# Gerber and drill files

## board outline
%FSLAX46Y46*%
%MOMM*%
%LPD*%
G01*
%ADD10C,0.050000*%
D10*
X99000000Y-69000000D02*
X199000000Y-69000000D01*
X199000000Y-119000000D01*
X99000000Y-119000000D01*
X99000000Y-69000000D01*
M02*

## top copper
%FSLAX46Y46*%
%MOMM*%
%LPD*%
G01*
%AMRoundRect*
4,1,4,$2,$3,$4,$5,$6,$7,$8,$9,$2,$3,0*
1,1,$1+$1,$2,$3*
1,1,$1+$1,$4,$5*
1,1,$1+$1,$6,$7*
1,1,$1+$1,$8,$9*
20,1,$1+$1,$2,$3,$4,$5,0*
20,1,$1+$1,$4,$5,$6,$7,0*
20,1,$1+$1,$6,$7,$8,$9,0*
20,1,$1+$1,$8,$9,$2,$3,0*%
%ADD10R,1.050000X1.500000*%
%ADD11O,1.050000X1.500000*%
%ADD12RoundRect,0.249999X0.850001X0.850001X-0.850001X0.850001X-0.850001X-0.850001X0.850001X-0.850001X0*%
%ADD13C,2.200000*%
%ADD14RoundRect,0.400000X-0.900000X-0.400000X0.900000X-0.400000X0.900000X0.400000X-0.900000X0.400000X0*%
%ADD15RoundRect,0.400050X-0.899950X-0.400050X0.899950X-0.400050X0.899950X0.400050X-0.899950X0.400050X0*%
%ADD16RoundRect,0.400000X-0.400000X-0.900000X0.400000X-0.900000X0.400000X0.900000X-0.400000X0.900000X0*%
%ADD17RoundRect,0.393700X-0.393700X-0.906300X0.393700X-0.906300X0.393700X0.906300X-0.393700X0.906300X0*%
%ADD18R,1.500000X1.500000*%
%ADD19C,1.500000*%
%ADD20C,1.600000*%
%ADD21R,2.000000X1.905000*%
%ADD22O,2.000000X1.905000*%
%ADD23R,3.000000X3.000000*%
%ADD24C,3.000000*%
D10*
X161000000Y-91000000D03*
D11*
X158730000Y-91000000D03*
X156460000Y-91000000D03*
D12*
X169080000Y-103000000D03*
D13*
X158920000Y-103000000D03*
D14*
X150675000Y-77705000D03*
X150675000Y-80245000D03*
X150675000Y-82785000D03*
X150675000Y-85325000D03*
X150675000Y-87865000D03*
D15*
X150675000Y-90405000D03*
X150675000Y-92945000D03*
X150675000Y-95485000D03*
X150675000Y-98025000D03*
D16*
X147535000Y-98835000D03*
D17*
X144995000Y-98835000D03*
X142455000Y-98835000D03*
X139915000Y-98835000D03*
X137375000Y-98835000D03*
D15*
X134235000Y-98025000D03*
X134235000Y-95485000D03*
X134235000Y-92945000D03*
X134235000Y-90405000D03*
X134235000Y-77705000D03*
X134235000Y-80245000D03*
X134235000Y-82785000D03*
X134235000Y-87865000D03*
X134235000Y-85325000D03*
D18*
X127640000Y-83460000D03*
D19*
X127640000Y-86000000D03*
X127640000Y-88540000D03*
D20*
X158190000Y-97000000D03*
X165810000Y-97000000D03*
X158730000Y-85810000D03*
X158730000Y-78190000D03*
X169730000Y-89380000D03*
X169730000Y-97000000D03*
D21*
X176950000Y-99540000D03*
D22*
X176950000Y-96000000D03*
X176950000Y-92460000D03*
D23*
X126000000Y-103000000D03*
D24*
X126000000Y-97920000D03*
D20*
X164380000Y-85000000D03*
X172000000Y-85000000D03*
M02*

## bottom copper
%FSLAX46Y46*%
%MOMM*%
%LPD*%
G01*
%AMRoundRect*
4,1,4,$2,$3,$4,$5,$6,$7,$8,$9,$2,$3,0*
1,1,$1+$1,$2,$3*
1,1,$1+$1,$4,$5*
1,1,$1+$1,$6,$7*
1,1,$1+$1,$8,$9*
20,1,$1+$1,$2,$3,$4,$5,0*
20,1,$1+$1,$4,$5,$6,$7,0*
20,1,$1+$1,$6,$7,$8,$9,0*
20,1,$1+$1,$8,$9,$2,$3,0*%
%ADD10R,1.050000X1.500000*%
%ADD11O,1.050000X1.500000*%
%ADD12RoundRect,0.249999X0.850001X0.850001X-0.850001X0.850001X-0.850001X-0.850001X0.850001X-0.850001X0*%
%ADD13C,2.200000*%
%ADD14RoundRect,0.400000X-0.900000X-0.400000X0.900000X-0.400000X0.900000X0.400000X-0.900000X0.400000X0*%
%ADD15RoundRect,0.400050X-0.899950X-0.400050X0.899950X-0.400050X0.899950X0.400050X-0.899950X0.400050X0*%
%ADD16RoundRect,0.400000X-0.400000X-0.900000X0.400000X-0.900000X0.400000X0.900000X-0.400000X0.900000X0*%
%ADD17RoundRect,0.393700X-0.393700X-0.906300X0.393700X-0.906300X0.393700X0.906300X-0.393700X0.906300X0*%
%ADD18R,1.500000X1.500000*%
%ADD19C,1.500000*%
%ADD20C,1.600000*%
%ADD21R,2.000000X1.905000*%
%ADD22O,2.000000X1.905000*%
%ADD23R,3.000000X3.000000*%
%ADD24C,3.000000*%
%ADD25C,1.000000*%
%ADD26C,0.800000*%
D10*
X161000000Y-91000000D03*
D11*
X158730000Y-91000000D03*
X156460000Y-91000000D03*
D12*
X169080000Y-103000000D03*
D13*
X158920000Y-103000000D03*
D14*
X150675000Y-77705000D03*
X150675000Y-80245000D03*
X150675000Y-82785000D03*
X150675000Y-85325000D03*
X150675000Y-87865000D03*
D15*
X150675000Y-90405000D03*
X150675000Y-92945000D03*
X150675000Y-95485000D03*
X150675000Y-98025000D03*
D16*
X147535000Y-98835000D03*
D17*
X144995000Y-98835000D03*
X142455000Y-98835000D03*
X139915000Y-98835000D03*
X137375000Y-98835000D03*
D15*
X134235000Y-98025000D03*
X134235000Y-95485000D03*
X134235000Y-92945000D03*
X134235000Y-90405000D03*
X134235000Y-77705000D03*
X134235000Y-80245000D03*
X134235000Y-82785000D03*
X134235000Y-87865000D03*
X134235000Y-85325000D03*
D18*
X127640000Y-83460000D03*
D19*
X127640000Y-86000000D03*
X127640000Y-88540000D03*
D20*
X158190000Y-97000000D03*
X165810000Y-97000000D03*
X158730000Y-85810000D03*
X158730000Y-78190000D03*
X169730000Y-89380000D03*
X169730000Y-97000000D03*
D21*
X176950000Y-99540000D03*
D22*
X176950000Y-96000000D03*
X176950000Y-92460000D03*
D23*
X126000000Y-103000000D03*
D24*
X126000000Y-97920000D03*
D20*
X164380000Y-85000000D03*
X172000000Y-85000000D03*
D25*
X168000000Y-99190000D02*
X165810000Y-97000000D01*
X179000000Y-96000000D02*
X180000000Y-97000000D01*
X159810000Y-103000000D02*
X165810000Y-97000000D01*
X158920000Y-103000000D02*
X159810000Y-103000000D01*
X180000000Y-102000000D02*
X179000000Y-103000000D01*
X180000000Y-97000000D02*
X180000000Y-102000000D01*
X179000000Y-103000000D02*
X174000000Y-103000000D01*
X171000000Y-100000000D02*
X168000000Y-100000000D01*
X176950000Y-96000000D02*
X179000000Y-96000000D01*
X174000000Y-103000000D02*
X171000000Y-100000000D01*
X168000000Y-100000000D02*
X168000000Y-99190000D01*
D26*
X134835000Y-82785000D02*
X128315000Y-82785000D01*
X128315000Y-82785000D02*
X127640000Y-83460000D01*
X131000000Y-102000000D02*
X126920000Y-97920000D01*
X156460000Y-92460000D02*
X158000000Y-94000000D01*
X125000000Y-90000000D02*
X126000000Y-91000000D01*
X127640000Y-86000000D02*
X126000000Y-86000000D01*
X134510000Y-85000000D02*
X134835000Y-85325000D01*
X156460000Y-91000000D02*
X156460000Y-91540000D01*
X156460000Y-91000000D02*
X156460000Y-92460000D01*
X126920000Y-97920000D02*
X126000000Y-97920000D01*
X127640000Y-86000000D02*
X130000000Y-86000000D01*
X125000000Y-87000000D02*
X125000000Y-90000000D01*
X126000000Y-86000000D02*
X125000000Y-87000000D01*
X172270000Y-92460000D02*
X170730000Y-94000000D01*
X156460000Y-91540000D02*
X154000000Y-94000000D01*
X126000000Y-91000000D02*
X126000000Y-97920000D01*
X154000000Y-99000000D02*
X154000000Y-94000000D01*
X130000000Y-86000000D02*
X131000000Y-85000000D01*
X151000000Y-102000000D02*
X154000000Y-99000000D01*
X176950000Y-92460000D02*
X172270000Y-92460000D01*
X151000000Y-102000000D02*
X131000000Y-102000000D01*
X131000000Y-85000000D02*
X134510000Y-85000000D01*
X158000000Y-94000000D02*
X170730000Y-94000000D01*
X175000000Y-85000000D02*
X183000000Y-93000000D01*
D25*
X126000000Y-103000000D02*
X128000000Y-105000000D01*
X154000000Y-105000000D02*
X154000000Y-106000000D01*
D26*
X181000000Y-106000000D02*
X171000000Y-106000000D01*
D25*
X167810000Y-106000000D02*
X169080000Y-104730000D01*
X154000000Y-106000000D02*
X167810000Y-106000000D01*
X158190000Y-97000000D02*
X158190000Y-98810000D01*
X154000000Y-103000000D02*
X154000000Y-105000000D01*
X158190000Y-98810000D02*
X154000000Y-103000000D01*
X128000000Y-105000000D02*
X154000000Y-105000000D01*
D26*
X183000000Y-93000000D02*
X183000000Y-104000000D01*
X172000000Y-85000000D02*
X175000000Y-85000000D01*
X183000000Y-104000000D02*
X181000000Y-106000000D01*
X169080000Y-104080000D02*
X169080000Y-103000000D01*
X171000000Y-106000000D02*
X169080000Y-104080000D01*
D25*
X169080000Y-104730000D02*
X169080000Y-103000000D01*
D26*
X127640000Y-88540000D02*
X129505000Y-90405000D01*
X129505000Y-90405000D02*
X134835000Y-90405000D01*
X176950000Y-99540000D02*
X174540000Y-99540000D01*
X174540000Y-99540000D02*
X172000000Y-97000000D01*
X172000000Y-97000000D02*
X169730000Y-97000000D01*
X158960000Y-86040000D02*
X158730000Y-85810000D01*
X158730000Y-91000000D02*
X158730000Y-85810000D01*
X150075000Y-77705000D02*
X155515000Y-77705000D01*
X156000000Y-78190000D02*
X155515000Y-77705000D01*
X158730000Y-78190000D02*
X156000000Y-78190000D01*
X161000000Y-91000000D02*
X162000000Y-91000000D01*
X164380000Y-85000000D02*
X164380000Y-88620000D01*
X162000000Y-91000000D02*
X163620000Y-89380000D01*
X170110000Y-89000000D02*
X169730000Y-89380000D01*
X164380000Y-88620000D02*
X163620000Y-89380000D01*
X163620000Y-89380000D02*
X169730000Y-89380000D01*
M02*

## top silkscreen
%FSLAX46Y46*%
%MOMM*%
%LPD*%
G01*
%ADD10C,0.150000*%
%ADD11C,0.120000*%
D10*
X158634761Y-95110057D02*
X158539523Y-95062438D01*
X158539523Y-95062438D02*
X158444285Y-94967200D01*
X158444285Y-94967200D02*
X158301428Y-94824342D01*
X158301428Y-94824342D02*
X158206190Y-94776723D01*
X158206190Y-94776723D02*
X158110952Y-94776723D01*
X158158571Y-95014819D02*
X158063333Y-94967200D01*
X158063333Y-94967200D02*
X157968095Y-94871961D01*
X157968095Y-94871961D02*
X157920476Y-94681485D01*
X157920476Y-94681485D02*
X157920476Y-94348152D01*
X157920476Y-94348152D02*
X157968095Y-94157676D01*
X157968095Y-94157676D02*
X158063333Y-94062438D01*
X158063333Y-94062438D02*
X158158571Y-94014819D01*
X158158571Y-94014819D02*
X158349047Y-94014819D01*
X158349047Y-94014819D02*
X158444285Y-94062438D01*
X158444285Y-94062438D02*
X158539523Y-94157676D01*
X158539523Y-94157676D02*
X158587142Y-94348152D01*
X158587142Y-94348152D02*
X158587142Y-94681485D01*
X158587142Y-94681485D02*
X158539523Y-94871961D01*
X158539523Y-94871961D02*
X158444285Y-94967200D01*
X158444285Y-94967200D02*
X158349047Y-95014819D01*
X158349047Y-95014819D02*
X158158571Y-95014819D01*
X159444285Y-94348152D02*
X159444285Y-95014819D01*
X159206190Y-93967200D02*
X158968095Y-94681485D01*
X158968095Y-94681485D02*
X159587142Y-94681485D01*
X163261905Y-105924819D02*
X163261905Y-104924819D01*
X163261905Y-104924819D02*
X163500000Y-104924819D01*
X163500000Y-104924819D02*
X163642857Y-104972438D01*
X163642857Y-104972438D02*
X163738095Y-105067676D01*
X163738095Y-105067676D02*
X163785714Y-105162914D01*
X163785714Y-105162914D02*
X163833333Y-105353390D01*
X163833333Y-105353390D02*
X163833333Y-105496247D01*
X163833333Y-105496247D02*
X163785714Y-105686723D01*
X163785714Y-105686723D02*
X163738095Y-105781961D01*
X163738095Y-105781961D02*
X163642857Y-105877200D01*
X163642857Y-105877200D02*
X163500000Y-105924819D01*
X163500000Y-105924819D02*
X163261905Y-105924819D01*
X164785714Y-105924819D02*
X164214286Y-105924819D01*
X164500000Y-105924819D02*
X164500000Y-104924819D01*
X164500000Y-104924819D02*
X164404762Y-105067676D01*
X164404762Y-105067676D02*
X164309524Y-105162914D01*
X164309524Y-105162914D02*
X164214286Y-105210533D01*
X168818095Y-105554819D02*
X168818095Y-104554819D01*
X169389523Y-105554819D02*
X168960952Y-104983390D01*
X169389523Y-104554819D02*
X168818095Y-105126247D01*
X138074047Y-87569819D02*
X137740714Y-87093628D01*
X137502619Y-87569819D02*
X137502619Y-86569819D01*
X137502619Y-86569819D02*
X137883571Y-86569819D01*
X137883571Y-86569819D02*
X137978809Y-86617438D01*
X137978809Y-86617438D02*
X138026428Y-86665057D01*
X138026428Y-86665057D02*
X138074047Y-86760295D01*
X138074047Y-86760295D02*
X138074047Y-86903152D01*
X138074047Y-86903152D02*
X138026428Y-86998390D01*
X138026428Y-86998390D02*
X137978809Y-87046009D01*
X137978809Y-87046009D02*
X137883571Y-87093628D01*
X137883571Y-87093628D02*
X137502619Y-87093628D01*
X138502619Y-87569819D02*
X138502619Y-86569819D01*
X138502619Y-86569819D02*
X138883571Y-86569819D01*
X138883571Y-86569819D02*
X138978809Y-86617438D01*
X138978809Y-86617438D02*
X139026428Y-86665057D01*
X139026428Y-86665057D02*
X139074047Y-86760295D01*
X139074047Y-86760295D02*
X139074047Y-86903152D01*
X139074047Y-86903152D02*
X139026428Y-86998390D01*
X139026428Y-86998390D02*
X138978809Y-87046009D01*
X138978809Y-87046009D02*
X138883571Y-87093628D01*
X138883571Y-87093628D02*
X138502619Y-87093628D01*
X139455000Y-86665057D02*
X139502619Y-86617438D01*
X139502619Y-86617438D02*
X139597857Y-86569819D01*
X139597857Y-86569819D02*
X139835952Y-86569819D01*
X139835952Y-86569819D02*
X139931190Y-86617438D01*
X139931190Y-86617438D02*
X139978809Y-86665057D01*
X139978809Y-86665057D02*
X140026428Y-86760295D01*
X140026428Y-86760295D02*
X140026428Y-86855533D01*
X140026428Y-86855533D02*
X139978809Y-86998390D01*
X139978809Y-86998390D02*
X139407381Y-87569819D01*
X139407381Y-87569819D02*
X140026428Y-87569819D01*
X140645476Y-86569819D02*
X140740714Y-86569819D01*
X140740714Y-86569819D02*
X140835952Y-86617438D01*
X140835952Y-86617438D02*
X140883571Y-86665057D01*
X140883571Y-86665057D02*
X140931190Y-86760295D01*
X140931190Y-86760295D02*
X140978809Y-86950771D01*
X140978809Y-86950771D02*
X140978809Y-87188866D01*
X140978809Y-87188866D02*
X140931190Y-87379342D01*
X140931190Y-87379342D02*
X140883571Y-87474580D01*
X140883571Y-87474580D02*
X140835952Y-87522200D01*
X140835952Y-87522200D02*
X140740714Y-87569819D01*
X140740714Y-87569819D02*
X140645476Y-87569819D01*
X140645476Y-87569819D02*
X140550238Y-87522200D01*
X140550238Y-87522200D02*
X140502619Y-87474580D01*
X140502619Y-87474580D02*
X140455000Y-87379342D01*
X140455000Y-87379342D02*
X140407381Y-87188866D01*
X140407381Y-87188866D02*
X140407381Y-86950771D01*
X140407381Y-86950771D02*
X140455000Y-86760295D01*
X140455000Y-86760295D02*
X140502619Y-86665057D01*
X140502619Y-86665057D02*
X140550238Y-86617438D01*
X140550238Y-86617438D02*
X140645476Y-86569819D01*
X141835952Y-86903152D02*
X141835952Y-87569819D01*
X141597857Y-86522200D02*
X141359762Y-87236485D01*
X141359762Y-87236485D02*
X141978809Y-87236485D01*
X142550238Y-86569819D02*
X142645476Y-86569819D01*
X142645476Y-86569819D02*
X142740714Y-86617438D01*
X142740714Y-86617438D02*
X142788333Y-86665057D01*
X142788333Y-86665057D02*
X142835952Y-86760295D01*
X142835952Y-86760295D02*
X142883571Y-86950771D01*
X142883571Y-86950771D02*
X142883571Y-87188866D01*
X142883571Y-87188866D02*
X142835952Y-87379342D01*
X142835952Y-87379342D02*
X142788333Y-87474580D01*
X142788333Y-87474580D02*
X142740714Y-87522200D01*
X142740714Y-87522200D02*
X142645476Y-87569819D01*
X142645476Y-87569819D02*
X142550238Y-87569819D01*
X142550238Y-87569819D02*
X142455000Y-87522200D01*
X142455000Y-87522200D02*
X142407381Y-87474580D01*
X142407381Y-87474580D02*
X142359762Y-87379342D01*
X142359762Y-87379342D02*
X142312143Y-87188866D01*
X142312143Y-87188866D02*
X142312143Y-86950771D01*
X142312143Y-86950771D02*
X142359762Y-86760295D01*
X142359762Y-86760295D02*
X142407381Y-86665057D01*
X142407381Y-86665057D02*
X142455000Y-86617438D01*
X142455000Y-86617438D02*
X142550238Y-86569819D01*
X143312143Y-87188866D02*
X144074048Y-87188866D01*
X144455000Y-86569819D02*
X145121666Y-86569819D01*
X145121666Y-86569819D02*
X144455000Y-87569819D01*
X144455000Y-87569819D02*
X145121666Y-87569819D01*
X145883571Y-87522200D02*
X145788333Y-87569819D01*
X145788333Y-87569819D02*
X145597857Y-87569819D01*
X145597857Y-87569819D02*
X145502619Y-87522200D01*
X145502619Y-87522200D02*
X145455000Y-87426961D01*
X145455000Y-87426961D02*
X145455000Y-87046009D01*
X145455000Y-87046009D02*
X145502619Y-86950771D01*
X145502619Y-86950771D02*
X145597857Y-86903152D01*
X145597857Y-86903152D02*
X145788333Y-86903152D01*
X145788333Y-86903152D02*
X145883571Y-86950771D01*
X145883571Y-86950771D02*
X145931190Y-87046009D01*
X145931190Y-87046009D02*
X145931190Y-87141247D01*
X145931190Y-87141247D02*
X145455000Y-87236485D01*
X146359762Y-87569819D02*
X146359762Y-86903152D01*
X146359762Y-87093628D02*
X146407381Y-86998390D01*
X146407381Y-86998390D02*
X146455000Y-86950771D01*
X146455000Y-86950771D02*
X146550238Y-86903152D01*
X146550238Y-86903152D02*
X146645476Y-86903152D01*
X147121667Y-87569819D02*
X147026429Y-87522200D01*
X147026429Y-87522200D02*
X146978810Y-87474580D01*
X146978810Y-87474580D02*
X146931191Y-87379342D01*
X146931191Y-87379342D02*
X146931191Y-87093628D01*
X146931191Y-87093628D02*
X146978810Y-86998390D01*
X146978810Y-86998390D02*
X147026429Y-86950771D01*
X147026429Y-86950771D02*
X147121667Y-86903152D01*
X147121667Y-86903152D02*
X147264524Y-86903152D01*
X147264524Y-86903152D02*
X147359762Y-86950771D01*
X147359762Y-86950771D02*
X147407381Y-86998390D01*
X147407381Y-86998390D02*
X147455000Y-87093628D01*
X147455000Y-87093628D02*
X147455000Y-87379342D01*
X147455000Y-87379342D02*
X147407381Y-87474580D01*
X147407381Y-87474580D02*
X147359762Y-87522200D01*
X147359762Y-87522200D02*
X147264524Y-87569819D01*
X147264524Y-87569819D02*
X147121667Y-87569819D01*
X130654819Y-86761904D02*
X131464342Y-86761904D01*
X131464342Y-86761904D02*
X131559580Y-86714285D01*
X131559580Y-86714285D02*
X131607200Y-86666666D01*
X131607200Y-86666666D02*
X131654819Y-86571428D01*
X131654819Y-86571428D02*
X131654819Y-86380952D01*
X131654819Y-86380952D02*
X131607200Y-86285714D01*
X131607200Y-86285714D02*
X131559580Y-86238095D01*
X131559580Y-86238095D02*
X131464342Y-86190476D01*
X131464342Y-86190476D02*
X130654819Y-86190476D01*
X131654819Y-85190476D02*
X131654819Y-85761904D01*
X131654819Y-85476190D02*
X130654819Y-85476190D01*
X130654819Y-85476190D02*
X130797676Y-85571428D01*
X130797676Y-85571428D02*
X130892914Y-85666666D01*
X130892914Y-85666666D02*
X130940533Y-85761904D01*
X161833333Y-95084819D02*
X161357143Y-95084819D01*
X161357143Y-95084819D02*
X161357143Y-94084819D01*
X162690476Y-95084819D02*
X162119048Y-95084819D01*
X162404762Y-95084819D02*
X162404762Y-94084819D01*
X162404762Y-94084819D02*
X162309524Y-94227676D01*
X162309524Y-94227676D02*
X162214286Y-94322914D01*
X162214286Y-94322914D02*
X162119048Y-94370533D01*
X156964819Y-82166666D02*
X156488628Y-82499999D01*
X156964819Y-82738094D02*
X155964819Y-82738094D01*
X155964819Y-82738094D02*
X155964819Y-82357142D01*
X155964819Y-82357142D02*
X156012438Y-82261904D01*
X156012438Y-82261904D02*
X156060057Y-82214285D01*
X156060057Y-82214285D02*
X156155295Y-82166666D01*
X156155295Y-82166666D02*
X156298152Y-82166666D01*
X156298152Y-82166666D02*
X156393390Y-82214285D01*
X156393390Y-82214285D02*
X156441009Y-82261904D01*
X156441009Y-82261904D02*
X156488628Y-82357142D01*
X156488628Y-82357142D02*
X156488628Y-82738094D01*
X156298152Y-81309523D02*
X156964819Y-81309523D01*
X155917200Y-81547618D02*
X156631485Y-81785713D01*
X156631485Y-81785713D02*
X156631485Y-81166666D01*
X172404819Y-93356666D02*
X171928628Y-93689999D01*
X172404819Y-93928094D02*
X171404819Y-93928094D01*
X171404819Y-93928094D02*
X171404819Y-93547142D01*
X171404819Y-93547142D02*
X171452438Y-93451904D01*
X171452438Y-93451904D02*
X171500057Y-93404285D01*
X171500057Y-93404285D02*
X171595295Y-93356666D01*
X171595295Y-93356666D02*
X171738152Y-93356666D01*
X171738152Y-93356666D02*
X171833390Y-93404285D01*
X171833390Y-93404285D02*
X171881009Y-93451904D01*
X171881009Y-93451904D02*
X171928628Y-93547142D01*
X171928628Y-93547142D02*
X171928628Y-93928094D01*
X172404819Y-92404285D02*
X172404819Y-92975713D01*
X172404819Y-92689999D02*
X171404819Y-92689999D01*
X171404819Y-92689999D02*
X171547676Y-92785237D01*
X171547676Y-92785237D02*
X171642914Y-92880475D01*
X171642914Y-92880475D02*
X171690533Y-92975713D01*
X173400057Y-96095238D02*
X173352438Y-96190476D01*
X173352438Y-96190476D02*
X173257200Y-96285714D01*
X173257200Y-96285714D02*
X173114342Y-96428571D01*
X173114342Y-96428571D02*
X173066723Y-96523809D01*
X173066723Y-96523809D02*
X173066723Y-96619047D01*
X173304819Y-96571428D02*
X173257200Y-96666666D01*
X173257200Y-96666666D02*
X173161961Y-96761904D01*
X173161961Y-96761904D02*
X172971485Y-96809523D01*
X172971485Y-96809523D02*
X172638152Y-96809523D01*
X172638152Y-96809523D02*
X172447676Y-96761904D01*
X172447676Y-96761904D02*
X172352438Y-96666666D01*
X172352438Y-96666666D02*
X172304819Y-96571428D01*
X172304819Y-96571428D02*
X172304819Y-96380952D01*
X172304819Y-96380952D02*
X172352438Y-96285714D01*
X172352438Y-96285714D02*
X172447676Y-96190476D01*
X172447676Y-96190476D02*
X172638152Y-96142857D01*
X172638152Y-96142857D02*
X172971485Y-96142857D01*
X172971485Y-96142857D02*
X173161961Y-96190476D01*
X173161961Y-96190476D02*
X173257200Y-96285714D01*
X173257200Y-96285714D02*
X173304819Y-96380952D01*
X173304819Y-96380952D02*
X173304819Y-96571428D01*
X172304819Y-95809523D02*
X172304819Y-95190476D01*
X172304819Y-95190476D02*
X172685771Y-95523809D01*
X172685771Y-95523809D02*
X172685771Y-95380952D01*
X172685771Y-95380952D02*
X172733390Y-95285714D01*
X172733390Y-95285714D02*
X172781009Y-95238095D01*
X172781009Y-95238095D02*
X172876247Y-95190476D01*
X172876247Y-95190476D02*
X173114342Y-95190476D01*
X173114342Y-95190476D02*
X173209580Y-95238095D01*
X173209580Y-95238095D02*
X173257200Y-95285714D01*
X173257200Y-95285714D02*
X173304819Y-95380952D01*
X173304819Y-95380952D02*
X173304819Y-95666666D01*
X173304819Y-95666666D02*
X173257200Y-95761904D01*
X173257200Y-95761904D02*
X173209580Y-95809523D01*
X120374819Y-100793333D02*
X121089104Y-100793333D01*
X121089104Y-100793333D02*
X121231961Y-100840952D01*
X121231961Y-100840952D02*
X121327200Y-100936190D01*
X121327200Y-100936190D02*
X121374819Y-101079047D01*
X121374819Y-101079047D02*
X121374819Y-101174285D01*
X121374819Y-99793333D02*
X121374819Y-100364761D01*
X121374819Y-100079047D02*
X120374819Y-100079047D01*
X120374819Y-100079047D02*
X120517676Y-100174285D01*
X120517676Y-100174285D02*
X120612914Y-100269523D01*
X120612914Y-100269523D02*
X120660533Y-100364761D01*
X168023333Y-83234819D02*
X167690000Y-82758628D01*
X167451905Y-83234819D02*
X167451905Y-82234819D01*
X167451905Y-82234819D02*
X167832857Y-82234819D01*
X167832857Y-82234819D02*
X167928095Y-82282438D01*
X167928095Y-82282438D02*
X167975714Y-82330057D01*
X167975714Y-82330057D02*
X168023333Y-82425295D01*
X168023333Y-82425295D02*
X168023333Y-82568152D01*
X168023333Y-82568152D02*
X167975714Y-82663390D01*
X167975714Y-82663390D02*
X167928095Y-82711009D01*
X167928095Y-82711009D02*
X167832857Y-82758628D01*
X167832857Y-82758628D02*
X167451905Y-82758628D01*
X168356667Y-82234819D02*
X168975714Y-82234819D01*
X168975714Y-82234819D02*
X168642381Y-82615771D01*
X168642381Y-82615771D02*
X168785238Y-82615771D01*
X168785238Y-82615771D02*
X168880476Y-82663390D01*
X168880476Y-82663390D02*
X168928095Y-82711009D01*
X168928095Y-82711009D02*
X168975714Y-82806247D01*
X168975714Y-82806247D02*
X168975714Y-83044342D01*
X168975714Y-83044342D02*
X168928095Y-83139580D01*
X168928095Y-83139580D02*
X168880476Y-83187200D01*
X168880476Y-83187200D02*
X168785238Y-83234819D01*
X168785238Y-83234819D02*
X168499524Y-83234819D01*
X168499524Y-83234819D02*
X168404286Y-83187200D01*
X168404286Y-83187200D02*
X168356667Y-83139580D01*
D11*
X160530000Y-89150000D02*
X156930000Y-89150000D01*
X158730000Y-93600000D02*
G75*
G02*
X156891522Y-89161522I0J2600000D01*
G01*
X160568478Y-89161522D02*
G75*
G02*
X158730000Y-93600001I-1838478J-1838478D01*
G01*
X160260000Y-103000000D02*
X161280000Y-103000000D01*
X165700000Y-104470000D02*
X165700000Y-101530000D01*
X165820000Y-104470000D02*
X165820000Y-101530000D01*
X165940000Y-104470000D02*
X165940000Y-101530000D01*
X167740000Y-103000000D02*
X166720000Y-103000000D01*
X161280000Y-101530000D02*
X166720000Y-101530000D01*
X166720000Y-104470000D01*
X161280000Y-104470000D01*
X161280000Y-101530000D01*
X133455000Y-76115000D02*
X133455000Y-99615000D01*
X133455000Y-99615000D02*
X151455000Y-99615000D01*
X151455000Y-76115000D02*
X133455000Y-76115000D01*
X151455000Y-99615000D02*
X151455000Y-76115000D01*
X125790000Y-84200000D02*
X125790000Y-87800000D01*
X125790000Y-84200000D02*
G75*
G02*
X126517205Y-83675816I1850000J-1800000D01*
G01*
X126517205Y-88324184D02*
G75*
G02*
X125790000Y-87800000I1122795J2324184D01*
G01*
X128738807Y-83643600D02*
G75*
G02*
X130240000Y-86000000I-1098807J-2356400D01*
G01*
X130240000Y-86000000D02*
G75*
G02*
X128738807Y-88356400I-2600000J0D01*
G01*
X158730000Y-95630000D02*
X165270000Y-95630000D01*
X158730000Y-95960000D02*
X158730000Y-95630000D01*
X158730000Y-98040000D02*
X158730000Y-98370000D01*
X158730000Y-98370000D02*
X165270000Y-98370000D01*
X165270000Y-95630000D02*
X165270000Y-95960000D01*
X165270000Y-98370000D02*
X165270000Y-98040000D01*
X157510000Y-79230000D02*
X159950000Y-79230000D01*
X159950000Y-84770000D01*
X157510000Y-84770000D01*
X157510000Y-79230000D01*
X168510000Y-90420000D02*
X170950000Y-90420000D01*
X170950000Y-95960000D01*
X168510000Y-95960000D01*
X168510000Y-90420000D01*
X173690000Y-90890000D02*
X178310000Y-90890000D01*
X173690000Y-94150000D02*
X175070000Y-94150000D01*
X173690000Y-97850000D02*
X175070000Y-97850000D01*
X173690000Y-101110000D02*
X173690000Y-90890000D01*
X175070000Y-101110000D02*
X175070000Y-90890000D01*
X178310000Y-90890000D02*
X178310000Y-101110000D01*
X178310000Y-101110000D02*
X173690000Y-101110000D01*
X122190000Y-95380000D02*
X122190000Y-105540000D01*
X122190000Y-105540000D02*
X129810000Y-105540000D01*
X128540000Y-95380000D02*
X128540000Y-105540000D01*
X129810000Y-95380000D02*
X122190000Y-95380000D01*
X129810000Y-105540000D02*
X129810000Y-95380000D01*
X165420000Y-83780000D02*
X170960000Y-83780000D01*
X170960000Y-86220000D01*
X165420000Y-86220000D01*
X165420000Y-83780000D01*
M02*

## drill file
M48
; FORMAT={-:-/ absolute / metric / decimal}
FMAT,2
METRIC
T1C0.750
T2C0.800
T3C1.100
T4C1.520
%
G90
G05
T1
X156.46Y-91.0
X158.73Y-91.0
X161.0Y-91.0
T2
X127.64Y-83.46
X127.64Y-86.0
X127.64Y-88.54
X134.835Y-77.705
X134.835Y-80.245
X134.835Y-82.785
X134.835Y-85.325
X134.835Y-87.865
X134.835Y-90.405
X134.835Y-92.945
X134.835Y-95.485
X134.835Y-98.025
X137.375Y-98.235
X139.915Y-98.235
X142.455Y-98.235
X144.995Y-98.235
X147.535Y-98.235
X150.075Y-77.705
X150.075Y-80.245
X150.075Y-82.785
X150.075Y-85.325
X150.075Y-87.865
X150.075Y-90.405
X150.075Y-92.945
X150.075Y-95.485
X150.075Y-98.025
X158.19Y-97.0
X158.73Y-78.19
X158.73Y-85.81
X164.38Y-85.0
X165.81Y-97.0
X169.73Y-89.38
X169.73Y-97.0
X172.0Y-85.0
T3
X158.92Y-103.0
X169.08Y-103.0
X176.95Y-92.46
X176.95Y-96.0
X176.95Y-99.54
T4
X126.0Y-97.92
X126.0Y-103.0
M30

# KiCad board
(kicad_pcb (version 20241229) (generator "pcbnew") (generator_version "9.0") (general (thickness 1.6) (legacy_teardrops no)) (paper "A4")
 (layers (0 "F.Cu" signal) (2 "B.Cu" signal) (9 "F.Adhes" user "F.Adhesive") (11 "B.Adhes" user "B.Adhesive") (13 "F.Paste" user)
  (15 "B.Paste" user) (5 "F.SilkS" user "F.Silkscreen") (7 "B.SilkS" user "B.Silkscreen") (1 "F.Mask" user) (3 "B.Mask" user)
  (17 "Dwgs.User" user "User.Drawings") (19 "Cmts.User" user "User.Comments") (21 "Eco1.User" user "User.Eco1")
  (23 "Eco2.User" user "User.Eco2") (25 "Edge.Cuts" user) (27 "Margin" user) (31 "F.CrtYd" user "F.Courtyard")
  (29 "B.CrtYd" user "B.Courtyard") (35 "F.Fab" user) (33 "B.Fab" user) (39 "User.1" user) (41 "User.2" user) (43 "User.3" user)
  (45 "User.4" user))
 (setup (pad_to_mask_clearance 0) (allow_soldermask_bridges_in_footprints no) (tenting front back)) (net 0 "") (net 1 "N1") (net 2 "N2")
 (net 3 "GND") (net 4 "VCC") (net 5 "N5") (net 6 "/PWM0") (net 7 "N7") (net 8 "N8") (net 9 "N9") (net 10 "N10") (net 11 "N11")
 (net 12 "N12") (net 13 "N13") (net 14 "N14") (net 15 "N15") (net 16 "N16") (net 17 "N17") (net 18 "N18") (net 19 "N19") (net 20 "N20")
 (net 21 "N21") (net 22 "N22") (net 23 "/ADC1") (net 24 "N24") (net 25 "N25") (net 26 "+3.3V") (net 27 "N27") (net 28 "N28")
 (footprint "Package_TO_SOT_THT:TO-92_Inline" (layer "F.Cu") (at 160 91 180)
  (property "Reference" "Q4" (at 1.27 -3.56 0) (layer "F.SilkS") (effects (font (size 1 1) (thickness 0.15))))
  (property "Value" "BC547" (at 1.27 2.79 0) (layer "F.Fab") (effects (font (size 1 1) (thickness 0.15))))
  (fp_line (start -0.53 1.85) (end 3.07 1.85) (stroke (width 0.12) (type solid)) (layer "F.SilkS"))
  (fp_arc (start 1.27 -2.6) (mid 3.672087 -0.994977) (end 3.108478 1.838478) (stroke (width 0.12) (type solid)) (layer "F.SilkS"))
  (fp_arc (start -0.568478 1.838478) (mid -1.132087 -0.994977) (end 1.27 -2.6) (stroke (width 0.12) (type solid)) (layer "F.SilkS"))
  (pad "1" thru_hole rect (at -1 0 180) (size 1.05 1.5) (drill 0.75) (layers "*.Cu" "*.Mask") (remove_unused_layers no) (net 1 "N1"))
  (pad "2" thru_hole oval (at 1.27 0 180) (size 1.05 1.5) (drill 0.75) (layers "*.Cu" "*.Mask") (remove_unused_layers no) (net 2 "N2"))
  (pad "3" thru_hole oval (at 3.54 0 180) (size 1.05 1.5) (drill 0.75) (layers "*.Cu" "*.Mask") (remove_unused_layers no) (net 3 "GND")))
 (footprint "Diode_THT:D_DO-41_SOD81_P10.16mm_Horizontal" (layer "F.Cu") (at 169.08 103 180)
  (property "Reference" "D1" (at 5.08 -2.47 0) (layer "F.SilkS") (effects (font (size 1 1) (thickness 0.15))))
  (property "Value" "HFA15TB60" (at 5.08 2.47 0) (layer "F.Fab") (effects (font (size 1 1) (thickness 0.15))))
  (fp_line (start 8.82 0) (end 7.8 0) (stroke (width 0.12) (type solid)) (layer "F.SilkS"))
  (fp_line (start 3.38 -1.47) (end 3.38 1.47) (stroke (width 0.12) (type solid)) (layer "F.SilkS"))
  (fp_line (start 3.26 -1.47) (end 3.26 1.47) (stroke (width 0.12) (type solid)) (layer "F.SilkS"))
  (fp_line (start 3.14 -1.47) (end 3.14 1.47) (stroke (width 0.12) (type solid)) (layer "F.SilkS"))
  (fp_line (start 1.34 0) (end 2.36 0) (stroke (width 0.12) (type solid)) (layer "F.SilkS"))
  (fp_rect (start 2.36 -1.47) (end 7.8 1.47) (stroke (width 0.12) (type solid)) (fill no) (layer "F.SilkS"))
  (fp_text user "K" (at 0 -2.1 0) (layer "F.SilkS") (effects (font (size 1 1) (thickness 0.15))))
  (pad "1" thru_hole roundrect (at 0 0 180) (size 2.2 2.2) (drill 1.1) (layers "*.Cu" "*.Mask") (remove_unused_layers no)
   (roundrect_rratio 0.113636) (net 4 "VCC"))
  (pad "2" thru_hole circle (at 10.16 0 180) (size 2.2 2.2) (drill 1.1) (layers "*.Cu" "*.Mask") (remove_unused_layers no) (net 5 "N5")))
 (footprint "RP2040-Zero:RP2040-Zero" (layer "F.Cu") (at 132.295 100.565)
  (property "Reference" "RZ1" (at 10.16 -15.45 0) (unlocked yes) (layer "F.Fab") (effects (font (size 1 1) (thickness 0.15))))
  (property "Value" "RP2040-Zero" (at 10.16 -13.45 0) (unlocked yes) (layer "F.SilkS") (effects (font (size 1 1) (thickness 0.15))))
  (fp_line (start 1.16 -24.45) (end 1.16 -0.95) (stroke (width 0.12) (type solid)) (layer "F.SilkS"))
  (fp_line (start 1.16 -0.95) (end 19.16 -0.95) (stroke (width 0.12) (type solid)) (layer "F.SilkS"))
  (fp_line (start 19.16 -24.45) (end 1.16 -24.45) (stroke (width 0.12) (type solid)) (layer "F.SilkS"))
  (fp_line (start 19.16 -0.95) (end 19.16 -24.45) (stroke (width 0.12) (type solid)) (layer "F.SilkS"))
  (pad "1" thru_hole roundrect (at 17.78 -22.86) (size 2.6 1.6) (drill 0.8 (offset 0.6 0)) (layers "*.Cu" "*.Mask")
   (remove_unused_layers no) (roundrect_rratio 0.25) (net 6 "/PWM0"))
  (pad "2" thru_hole roundrect (at 17.78 -20.32) (size 2.6 1.6) (drill 0.8 (offset 0.6 0)) (layers "*.Cu" "*.Mask")
   (remove_unused_layers no) (roundrect_rratio 0.25) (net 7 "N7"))
  (pad "3" thru_hole roundrect (at 17.78 -17.78) (size 2.6 1.6) (drill 0.8 (offset 0.6 0)) (layers "*.Cu" "*.Mask")
   (remove_unused_layers no) (roundrect_rratio 0.25) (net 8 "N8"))
  (pad "4" thru_hole roundrect (at 17.78 -15.24) (size 2.6 1.6) (drill 0.8 (offset 0.6 0)) (layers "*.Cu" "*.Mask")
   (remove_unused_layers no) (roundrect_rratio 0.25) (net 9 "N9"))
  (pad "5" thru_hole roundrect (at 17.78 -12.7) (size 2.6 1.6) (drill 0.8 (offset 0.6 0)) (layers "*.Cu" "*.Mask") (remove_unused_layers no)
   (roundrect_rratio 0.25) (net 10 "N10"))
  (pad "6" thru_hole roundrect (at 17.78 -10.16) (size 2.6 1.6002) (drill 0.8 (offset 0.6 0)) (layers "*.Cu" "*.Mask")
   (remove_unused_layers no) (roundrect_rratio 0.25) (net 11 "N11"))
  (pad "7" thru_hole roundrect (at 17.78 -7.62) (size 2.6 1.6002) (drill 0.8 (offset 0.6 0)) (layers "*.Cu" "*.Mask")
   (remove_unused_layers no) (roundrect_rratio 0.25) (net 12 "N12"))
  (pad "8" thru_hole roundrect (at 17.78 -5.08) (size 2.6 1.6002) (drill 0.8 (offset 0.6 0)) (layers "*.Cu" "*.Mask")
   (remove_unused_layers no) (roundrect_rratio 0.25) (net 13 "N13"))
  (pad "9" thru_hole roundrect (at 17.78 -2.54) (size 2.6 1.6002) (drill 0.8 (offset 0.6 0)) (layers "*.Cu" "*.Mask")
   (remove_unused_layers no) (roundrect_rratio 0.25) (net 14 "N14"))
  (pad "10" thru_hole roundrect (at 15.24 -2.33) (size 1.6 2.6) (drill 0.8 (offset 0 0.6)) (layers "*.Cu" "*.Mask")
   (remove_unused_layers no) (roundrect_rratio 0.25) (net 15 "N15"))
  (pad "11" thru_hole roundrect (at 12.7 -2.33) (size 1.5748 2.6) (drill 0.8 (offset 0 0.6)) (layers "*.Cu" "*.Mask")
   (remove_unused_layers no) (roundrect_rratio 0.25) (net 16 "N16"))
  (pad "12" thru_hole roundrect (at 10.16 -2.33) (size 1.5748 2.6) (drill 0.8 (offset 0 0.6)) (layers "*.Cu" "*.Mask")
   (remove_unused_layers no) (roundrect_rratio 0.25) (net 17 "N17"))
  (pad "13" thru_hole roundrect (at 7.62 -2.33) (size 1.5748 2.6) (drill 0.8 (offset 0 0.6)) (layers "*.Cu" "*.Mask")
   (remove_unused_layers no) (roundrect_rratio 0.25) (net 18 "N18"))
  (pad "14" thru_hole roundrect (at 5.08 -2.33) (size 1.5748 2.6) (drill 0.8 (offset 0 0.6)) (layers "*.Cu" "*.Mask")
   (remove_unused_layers no) (roundrect_rratio 0.25) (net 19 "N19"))
  (pad "15" thru_hole roundrect (at 2.54 -2.54) (size 2.6 1.6002) (drill 0.8 (offset -0.6 0)) (layers "*.Cu" "*.Mask")
   (remove_unused_layers no) (roundrect_rratio 0.25) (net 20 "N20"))
  (pad "16" thru_hole roundrect (at 2.54 -5.08) (size 2.6 1.6002) (drill 0.8 (offset -0.6 0)) (layers "*.Cu" "*.Mask")
   (remove_unused_layers no) (roundrect_rratio 0.25) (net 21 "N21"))
  (pad "17" thru_hole roundrect (at 2.54 -7.62) (size 2.6 1.6002) (drill 0.8 (offset -0.6 0)) (layers "*.Cu" "*.Mask")
   (remove_unused_layers no) (roundrect_rratio 0.25) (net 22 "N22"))
  (pad "18" thru_hole roundrect (at 2.54 -10.16) (size 2.6 1.6002) (drill 0.8 (offset -0.6 0)) (layers "*.Cu" "*.Mask")
   (remove_unused_layers no) (roundrect_rratio 0.25) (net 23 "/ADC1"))
  (pad "19" thru_hole roundrect (at 2.54 -22.86) (size 2.6 1.6002) (drill 0.8 (offset -0.6 0)) (layers "*.Cu" "*.Mask")
   (remove_unused_layers no) (roundrect_rratio 0.25) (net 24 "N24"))
  (pad "20" thru_hole roundrect (at 2.54 -20.32) (size 2.6 1.6002) (drill 0.8 (offset -0.6 0)) (layers "*.Cu" "*.Mask")
   (remove_unused_layers no) (roundrect_rratio 0.25) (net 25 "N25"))
  (pad "21" thru_hole roundrect (at 2.54 -17.78) (size 2.6 1.6002) (drill 0.8 (offset -0.6 0)) (layers "*.Cu" "*.Mask")
   (remove_unused_layers no) (roundrect_rratio 0.25) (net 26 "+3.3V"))
  (pad "22" thru_hole roundrect (at 2.54 -12.7) (size 2.6 1.6002) (drill 0.8 (offset -0.6 0)) (layers "*.Cu" "*.Mask")
   (remove_unused_layers no) (roundrect_rratio 0.25) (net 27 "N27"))
  (pad "23" thru_hole roundrect (at 2.54 -15.24) (size 2.6 1.6002) (drill 0.8 (offset -0.6 0)) (layers "*.Cu" "*.Mask")
   (remove_unused_layers no) (roundrect_rratio 0.25) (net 3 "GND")))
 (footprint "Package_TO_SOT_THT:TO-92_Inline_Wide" (layer "F.Cu") (at 127.64 83.46 -90)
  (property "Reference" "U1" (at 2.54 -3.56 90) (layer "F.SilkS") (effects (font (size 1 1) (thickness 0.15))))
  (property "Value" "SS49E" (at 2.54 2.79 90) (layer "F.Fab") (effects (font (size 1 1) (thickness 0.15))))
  (fp_line (start 0.74 1.85) (end 4.34 1.85) (stroke (width 0.12) (type solid)) (layer "F.SilkS"))
  (fp_arc (start 0.74 1.85) (mid 0.446097 1.509328) (end 0.215816 1.122795) (stroke (width 0.12) (type solid)) (layer "F.SilkS"))
  (fp_arc (start 4.864184 1.122795) (mid 4.633903 1.509328) (end 4.34 1.85) (stroke (width 0.12) (type solid)) (layer "F.SilkS"))
  (fp_arc (start 0.1836 -1.098807) (mid 1.143021 -2.192817) (end 2.54 -2.6) (stroke (width 0.12) (type solid)) (layer "F.SilkS"))
  (fp_arc (start 2.54 -2.6) (mid 3.936979 -2.192818) (end 4.8964 -1.098807) (stroke (width 0.12) (type solid)) (layer "F.SilkS"))
  (pad "1" thru_hole rect (at 0 0 270) (size 1.5 1.5) (drill 0.8) (layers "*.Cu" "*.Mask") (remove_unused_layers no) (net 26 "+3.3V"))
  (pad "2" thru_hole circle (at 2.54 0 270) (size 1.5 1.5) (drill 0.8) (layers "*.Cu" "*.Mask") (remove_unused_layers no) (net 3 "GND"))
  (pad "3" thru_hole circle (at 5.08 0 270) (size 1.5 1.5) (drill 0.8) (layers "*.Cu" "*.Mask") (remove_unused_layers no) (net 23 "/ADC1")))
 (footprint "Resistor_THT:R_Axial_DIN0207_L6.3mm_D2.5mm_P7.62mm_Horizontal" (layer "F.Cu") (at 158.19 97)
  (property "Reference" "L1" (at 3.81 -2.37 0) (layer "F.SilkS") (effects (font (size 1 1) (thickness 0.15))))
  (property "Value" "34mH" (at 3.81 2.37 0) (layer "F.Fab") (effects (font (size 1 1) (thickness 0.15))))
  (fp_line (start 0.54 -1.37) (end 7.08 -1.37) (stroke (width 0.12) (type solid)) (layer "F.SilkS"))
  (fp_line (start 0.54 -1.04) (end 0.54 -1.37) (stroke (width 0.12) (type solid)) (layer "F.SilkS"))
  (fp_line (start 0.54 1.04) (end 0.54 1.37) (stroke (width 0.12) (type solid)) (layer "F.SilkS"))
  (fp_line (start 0.54 1.37) (end 7.08 1.37) (stroke (width 0.12) (type solid)) (layer "F.SilkS"))
  (fp_line (start 7.08 -1.37) (end 7.08 -1.04) (stroke (width 0.12) (type solid)) (layer "F.SilkS"))
  (fp_line (start 7.08 1.37) (end 7.08 1.04) (stroke (width 0.12) (type solid)) (layer "F.SilkS"))
  (pad "1" thru_hole circle (at 0 0) (size 1.6 1.6) (drill 0.8) (layers "*.Cu" "*.Mask") (remove_unused_layers no) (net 4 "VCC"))
  (pad "2" thru_hole circle (at 7.62 0) (size 1.6 1.6) (drill 0.8) (layers "*.Cu" "*.Mask") (remove_unused_layers no) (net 5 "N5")))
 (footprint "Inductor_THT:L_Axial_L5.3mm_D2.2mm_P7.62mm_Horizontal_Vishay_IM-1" (layer "F.Cu") (at 158.73 85.81 90)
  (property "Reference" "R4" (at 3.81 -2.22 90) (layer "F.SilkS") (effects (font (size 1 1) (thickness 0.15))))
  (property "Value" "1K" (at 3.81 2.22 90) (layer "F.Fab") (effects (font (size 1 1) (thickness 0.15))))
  (fp_rect (start 1.04 -1.22) (end 6.58 1.22) (stroke (width 0.12) (type solid)) (fill no) (layer "F.SilkS"))
  (pad "1" thru_hole circle (at 0 0 90) (size 1.6 1.6) (drill 0.8) (layers "*.Cu" "*.Mask") (remove_unused_layers no) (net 2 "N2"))
  (pad "2" thru_hole circle (at 7.62 0 90) (size 1.6 1.6) (drill 0.8) (layers "*.Cu" "*.Mask") (remove_unused_layers no) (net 6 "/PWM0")))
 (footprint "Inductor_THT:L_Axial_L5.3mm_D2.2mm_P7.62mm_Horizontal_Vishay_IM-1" (layer "F.Cu") (at 169.73 89.38 -90)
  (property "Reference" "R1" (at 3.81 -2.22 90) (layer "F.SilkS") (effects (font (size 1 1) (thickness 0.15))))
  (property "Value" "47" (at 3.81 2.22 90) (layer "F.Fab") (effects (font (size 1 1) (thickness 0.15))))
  (fp_rect (start 1.04 -1.22) (end 6.58 1.22) (stroke (width 0.12) (type solid)) (fill no) (layer "F.SilkS"))
  (pad "1" thru_hole circle (at 0 0 270) (size 1.6 1.6) (drill 0.8) (layers "*.Cu" "*.Mask") (remove_unused_layers no) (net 1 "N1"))
  (pad "2" thru_hole circle (at 7.62 0 270) (size 1.6 1.6) (drill 0.8) (layers "*.Cu" "*.Mask") (remove_unused_layers no) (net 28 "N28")))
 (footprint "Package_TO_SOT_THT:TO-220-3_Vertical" (layer "F.Cu") (at 176.95 98.54 90)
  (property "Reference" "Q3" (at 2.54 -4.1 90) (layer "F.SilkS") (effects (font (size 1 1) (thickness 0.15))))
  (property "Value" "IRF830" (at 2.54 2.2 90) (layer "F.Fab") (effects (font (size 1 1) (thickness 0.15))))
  (fp_line (start 7.65 -3.26) (end 7.65 1.36) (stroke (width 0.12) (type solid)) (layer "F.SilkS"))
  (fp_line (start 4.39 -3.26) (end 4.39 -1.88) (stroke (width 0.12) (type solid)) (layer "F.SilkS"))
  (fp_line (start 0.69 -3.26) (end 0.69 -1.88) (stroke (width 0.12) (type solid)) (layer "F.SilkS"))
  (fp_line (start -2.57 -3.26) (end 7.65 -3.26) (stroke (width 0.12) (type solid)) (layer "F.SilkS"))
  (fp_line (start -2.57 -1.88) (end 7.65 -1.88) (stroke (width 0.12) (type solid)) (layer "F.SilkS"))
  (fp_line (start 7.65 1.36) (end -2.57 1.36) (stroke (width 0.12) (type solid)) (layer "F.SilkS"))
  (fp_line (start -2.57 1.36) (end -2.57 -3.26) (stroke (width 0.12) (type solid)) (layer "F.SilkS"))
  (pad "1" thru_hole rect (at -1 0 90) (size 1.905 2) (drill 1.1) (layers "*.Cu" "*.Mask") (remove_unused_layers no) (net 28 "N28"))
  (pad "2" thru_hole oval (at 2.54 0 90) (size 1.905 2) (drill 1.1) (layers "*.Cu" "*.Mask") (remove_unused_layers no) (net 5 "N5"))
  (pad "3" thru_hole oval (at 6.08 0 90) (size 1.905 2) (drill 1.1) (layers "*.Cu" "*.Mask") (remove_unused_layers no) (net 3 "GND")))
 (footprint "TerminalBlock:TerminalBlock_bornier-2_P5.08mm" (layer "F.Cu") (at 126 103 90)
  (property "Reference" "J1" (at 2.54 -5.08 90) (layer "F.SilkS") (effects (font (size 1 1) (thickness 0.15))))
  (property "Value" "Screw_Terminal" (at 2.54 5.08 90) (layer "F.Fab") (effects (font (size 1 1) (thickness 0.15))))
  (fp_line (start 7.62 -3.81) (end -2.54 -3.81) (stroke (width 0.12) (type solid)) (layer "F.SilkS"))
  (fp_line (start -2.54 -3.81) (end -2.54 3.81) (stroke (width 0.12) (type solid)) (layer "F.SilkS"))
  (fp_line (start 7.62 2.54) (end -2.54 2.54) (stroke (width 0.12) (type solid)) (layer "F.SilkS"))
  (fp_line (start 7.62 3.81) (end 7.62 -3.81) (stroke (width 0.12) (type solid)) (layer "F.SilkS"))
  (fp_line (start -2.54 3.81) (end 7.62 3.81) (stroke (width 0.12) (type solid)) (layer "F.SilkS"))
  (pad "1" thru_hole rect (at 0 0 90) (size 3 3) (drill 1.52) (layers "*.Cu" "*.Mask") (remove_unused_layers no) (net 4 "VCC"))
  (pad "2" thru_hole circle (at 5.08 0 90) (size 3 3) (drill 1.52) (layers "*.Cu" "*.Mask") (remove_unused_layers no) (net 3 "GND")))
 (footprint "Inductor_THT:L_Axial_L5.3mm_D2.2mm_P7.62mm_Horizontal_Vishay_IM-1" (layer "F.Cu") (at 164.38 85)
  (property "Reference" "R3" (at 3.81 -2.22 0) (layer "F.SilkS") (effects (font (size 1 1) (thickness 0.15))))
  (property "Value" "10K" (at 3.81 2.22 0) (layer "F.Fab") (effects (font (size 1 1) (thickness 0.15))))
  (fp_rect (start 1.04 -1.22) (end 6.58 1.22) (stroke (width 0.12) (type solid)) (fill no) (layer "F.SilkS"))
  (pad "1" thru_hole circle (at 0 0) (size 1.6 1.6) (drill 0.8) (layers "*.Cu" "*.Mask") (remove_unused_layers no) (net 1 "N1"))
  (pad "2" thru_hole circle (at 7.62 0) (size 1.6 1.6) (drill 0.8) (layers "*.Cu" "*.Mask") (remove_unused_layers no) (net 4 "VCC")))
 (gr_rect (start 99 69) (end 199 119) (stroke (width 0.05) (type default)) (fill no) (layer "Edge.Cuts"))
 (segment (start 168 99.19) (end 165.81 97) (width 1) (layer "B.Cu") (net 5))
 (segment (start 179 96) (end 180 97) (width 1) (layer "B.Cu") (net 5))
 (segment (start 159.81 103) (end 165.81 97) (width 1) (layer "B.Cu") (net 5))
 (segment (start 158.92 103) (end 159.81 103) (width 1) (layer "B.Cu") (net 5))
 (segment (start 180 102) (end 179 103) (width 1) (layer "B.Cu") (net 5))
 (segment (start 180 97) (end 180 102) (width 1) (layer "B.Cu") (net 5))
 (segment (start 179 103) (end 174 103) (width 1) (layer "B.Cu") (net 5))
 (segment (start 171 100) (end 168 100) (width 1) (layer "B.Cu") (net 5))
 (segment (start 176.95 96) (end 179 96) (width 1) (layer "B.Cu") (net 5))
 (segment (start 174 103) (end 171 100) (width 1) (layer "B.Cu") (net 5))
 (segment (start 168 100) (end 168 99.19) (width 1) (layer "B.Cu") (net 5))
 (segment (start 134.835 82.785) (end 128.315 82.785) (width 0.8) (layer "B.Cu") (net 26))
 (segment (start 128.315 82.785) (end 127.64 83.46) (width 0.8) (layer "B.Cu") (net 26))
 (segment (start 131 102) (end 126.92 97.92) (width 0.8) (layer "B.Cu") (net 3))
 (segment (start 156.46 92.46) (end 158 94) (width 0.8) (layer "B.Cu") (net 3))
 (segment (start 125 90) (end 126 91) (width 0.8) (layer "B.Cu") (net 3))
 (segment (start 127.64 86) (end 126 86) (width 0.8) (layer "B.Cu") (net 3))
 (segment (start 134.51 85) (end 134.835 85.325) (width 0.8) (layer "B.Cu") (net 3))
 (segment (start 156.46 91) (end 156.46 91.54) (width 0.8) (layer "B.Cu") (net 3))
 (segment (start 156.46 91) (end 156.46 92.46) (width 0.8) (layer "B.Cu") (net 3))
 (segment (start 126.92 97.92) (end 126 97.92) (width 0.8) (layer "B.Cu") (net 3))
 (segment (start 127.64 86) (end 130 86) (width 0.8) (layer "B.Cu") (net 3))
 (segment (start 125 87) (end 125 90) (width 0.8) (layer "B.Cu") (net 3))
 (segment (start 126 86) (end 125 87) (width 0.8) (layer "B.Cu") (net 3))
 (segment (start 172.27 92.46) (end 170.73 94) (width 0.8) (layer "B.Cu") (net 3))
 (segment (start 156.46 91.54) (end 154 94) (width 0.8) (layer "B.Cu") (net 3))
 (segment (start 126 91) (end 126 97.92) (width 0.8) (layer "B.Cu") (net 3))
 (segment (start 154 99) (end 154 94) (width 0.8) (layer "B.Cu") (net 3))
 (segment (start 130 86) (end 131 85) (width 0.8) (layer "B.Cu") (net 3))
 (segment (start 151 102) (end 154 99) (width 0.8) (layer "B.Cu") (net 3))
 (segment (start 176.95 92.46) (end 172.27 92.46) (width 0.8) (layer "B.Cu") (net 3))
 (segment (start 151 102) (end 131 102) (width 0.8) (layer "B.Cu") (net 3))
 (segment (start 131 85) (end 134.51 85) (width 0.8) (layer "B.Cu") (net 3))
 (segment (start 158 94) (end 170.73 94) (width 0.8) (layer "B.Cu") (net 3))
 (segment (start 175 85) (end 183 93) (width 0.8) (layer "B.Cu") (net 4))
 (segment (start 126 103) (end 128 105) (width 1) (layer "B.Cu") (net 4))
 (segment (start 154 105) (end 154 106) (width 1) (layer "B.Cu") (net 4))
 (segment (start 181 106) (end 171 106) (width 0.8) (layer "B.Cu") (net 4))
 (segment (start 167.81 106) (end 169.08 104.73) (width 1) (layer "B.Cu") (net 4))
 (segment (start 154 106) (end 167.81 106) (width 1) (layer "B.Cu") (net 4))
 (segment (start 158.19 97) (end 158.19 98.81) (width 1) (layer "B.Cu") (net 4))
 (segment (start 154 103) (end 154 105) (width 1) (layer "B.Cu") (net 4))
 (segment (start 158.19 98.81) (end 154 103) (width 1) (layer "B.Cu") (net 4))
 (segment (start 128 105) (end 154 105) (width 1) (layer "B.Cu") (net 4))
 (segment (start 183 93) (end 183 104) (width 0.8) (layer "B.Cu") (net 4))
 (segment (start 172 85) (end 175 85) (width 0.8) (layer "B.Cu") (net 4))
 (segment (start 183 104) (end 181 106) (width 0.8) (layer "B.Cu") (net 4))
 (segment (start 169.08 104.08) (end 169.08 103) (width 0.8) (layer "B.Cu") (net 4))
 (segment (start 171 106) (end 169.08 104.08) (width 0.8) (layer "B.Cu") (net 4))
 (segment (start 169.08 104.73) (end 169.08 103) (width 1) (layer "B.Cu") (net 4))
 (segment (start 127.64 88.54) (end 129.505 90.405) (width 0.8) (layer "B.Cu") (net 23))
 (segment (start 129.505 90.405) (end 134.835 90.405) (width 0.8) (layer "B.Cu") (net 23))
 (segment (start 176.95 99.54) (end 174.54 99.54) (width 0.8) (layer "B.Cu") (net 28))
 (segment (start 174.54 99.54) (end 172 97) (width 0.8) (layer "B.Cu") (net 28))
 (segment (start 172 97) (end 169.73 97) (width 0.8) (layer "B.Cu") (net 28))
 (segment (start 158.96 86.04) (end 158.73 85.81) (width 0.8) (layer "B.Cu") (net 2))
 (segment (start 158.73 91) (end 158.73 85.81) (width 0.8) (layer "B.Cu") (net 2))
 (segment (start 150.075 77.705) (end 155.515 77.705) (width 0.8) (layer "B.Cu") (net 6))
 (segment (start 156 78.19) (end 155.515 77.705) (width 0.8) (layer "B.Cu") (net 6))
 (segment (start 158.73 78.19) (end 156 78.19) (width 0.8) (layer "B.Cu") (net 6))
 (segment (start 161 91) (end 162 91) (width 0.8) (layer "B.Cu") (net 1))
 (segment (start 164.38 85) (end 164.38 88.62) (width 0.8) (layer "B.Cu") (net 1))
 (segment (start 162 91) (end 163.62 89.38) (width 0.8) (layer "B.Cu") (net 1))
 (segment (start 170.11 89) (end 169.73 89.38) (width 0.8) (layer "B.Cu") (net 1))
 (segment (start 164.38 88.62) (end 163.62 89.38) (width 0.8) (layer "B.Cu") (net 1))
 (segment (start 163.62 89.38) (end 169.73 89.38) (width 0.8) (layer "B.Cu") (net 1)))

